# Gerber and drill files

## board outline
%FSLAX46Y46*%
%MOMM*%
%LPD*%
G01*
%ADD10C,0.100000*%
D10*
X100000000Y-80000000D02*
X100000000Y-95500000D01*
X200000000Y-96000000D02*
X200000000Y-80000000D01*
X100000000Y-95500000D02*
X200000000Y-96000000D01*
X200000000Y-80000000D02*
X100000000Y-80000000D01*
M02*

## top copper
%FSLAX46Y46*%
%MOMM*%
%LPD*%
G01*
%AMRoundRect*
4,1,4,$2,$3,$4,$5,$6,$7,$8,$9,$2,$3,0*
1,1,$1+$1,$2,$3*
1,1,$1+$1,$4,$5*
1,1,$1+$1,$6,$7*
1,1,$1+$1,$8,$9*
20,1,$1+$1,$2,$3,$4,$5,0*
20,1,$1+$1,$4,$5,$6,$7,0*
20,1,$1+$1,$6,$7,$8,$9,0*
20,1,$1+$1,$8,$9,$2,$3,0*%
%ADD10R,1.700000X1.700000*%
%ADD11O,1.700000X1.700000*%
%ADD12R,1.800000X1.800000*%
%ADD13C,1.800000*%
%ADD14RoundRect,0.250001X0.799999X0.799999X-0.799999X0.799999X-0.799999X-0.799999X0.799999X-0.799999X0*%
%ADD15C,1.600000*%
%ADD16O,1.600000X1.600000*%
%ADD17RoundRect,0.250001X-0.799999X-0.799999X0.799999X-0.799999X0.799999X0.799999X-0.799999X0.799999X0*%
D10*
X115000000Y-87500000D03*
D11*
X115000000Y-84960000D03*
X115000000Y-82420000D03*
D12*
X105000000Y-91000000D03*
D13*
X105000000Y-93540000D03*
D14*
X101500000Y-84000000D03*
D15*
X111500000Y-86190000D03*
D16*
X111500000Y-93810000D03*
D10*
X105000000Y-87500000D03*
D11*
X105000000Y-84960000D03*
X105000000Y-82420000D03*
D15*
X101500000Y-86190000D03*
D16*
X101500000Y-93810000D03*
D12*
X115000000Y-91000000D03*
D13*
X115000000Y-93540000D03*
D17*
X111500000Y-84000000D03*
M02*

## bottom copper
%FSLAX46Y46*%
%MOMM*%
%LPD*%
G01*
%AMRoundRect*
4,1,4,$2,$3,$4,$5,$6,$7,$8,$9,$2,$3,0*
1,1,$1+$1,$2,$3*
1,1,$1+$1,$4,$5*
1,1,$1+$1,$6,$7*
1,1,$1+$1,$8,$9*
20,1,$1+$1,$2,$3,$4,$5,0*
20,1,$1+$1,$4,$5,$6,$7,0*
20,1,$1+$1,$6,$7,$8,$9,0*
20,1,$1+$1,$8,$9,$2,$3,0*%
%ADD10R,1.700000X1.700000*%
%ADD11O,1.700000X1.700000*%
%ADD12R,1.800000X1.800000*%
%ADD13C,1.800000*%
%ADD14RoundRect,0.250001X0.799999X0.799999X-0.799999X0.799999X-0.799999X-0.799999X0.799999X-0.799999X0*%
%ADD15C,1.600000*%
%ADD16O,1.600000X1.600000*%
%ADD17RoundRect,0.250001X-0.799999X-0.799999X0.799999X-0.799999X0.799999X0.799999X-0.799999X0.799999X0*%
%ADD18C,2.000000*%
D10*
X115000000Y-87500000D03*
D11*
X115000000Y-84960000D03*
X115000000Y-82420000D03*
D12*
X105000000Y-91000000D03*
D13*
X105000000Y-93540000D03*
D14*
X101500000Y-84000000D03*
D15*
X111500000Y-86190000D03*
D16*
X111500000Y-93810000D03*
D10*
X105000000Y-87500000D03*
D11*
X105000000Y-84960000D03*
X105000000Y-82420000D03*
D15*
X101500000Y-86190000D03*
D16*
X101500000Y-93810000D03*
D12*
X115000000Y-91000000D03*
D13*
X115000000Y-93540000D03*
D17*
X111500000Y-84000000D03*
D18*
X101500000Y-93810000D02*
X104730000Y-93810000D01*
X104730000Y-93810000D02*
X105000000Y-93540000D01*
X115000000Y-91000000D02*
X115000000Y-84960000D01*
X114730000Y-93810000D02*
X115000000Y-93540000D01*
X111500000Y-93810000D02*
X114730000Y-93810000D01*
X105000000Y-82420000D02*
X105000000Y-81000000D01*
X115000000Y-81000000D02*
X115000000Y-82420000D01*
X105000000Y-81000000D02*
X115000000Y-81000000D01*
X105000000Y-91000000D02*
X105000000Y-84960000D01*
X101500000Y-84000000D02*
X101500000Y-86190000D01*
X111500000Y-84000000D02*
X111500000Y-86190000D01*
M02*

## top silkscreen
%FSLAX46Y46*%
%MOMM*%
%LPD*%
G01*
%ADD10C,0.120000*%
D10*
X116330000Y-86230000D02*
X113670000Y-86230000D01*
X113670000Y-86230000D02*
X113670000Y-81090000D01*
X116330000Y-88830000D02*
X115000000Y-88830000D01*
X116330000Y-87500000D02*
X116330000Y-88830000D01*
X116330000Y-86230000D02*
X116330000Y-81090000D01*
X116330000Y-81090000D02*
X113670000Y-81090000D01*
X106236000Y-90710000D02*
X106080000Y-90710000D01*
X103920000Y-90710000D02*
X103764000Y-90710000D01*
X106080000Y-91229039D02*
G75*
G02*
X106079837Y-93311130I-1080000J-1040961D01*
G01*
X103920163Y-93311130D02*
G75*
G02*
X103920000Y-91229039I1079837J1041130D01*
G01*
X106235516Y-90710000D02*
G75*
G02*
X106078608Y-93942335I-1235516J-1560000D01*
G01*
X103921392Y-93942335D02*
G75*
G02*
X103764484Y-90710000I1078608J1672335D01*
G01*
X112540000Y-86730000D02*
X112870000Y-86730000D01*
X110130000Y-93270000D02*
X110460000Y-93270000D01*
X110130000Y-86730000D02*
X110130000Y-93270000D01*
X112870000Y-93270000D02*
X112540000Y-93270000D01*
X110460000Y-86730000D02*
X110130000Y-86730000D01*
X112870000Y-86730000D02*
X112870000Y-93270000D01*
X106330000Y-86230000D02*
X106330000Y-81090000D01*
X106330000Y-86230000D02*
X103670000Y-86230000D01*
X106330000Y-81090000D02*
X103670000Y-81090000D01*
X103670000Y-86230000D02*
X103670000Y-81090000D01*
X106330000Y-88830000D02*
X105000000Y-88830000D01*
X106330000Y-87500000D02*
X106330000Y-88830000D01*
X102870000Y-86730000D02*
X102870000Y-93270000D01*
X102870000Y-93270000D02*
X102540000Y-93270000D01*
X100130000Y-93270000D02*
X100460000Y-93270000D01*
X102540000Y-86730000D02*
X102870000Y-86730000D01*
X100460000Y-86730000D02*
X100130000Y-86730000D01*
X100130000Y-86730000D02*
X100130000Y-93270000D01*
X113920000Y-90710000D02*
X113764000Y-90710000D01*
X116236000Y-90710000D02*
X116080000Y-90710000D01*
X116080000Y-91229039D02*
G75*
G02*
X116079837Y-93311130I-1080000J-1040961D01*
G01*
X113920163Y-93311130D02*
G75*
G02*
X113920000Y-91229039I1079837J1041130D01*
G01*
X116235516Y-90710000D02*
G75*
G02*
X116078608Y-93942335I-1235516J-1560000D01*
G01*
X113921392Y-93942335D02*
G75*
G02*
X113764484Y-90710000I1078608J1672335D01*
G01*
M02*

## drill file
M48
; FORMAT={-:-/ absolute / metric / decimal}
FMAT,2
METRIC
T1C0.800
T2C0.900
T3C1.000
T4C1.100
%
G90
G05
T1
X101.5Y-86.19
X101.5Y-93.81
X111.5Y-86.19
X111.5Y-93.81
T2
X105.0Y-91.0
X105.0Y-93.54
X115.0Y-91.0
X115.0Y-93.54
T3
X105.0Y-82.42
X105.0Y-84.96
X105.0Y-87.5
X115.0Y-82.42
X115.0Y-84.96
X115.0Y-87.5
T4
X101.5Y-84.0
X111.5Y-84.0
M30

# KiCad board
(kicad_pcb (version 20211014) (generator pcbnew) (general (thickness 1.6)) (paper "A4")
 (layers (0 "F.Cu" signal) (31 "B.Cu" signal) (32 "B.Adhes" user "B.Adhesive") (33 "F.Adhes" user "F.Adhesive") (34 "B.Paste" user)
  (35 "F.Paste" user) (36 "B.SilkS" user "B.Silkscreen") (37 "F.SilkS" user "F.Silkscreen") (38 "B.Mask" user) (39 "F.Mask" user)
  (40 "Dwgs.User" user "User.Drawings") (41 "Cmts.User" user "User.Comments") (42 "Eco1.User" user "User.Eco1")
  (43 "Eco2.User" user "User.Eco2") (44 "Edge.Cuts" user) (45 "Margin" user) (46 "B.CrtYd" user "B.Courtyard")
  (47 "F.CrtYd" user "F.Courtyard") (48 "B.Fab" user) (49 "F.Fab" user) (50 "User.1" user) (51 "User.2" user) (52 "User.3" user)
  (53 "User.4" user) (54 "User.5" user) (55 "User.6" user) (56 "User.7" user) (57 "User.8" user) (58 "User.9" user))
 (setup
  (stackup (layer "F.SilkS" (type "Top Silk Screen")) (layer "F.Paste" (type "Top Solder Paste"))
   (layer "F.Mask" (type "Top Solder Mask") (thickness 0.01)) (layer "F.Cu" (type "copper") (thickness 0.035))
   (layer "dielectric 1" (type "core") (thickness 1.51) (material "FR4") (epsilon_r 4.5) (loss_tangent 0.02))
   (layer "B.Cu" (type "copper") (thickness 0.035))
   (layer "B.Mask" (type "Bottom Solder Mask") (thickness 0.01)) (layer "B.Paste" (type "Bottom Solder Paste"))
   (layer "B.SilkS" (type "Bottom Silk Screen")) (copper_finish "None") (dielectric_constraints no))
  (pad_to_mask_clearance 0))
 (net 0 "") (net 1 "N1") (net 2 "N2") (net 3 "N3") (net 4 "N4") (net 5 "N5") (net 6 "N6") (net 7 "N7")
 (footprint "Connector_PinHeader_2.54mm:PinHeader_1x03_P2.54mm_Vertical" (layer "F.Cu") (at 115 87.5 180)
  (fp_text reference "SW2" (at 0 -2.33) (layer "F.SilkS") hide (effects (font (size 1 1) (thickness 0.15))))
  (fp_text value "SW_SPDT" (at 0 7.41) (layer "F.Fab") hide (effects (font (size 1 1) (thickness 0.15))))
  (fp_line (start -1.33 1.27) (end 1.33 1.27) (layer "F.SilkS") (width 0.12))
  (fp_line (start 1.33 1.27) (end 1.33 6.41) (layer "F.SilkS") (width 0.12))
  (fp_line (start -1.33 -1.33) (end 0 -1.33) (layer "F.SilkS") (width 0.12))
  (fp_line (start -1.33 0) (end -1.33 -1.33) (layer "F.SilkS") (width 0.12))
  (fp_line (start -1.33 1.27) (end -1.33 6.41) (layer "F.SilkS") (width 0.12))
  (fp_line (start -1.33 6.41) (end 1.33 6.41) (layer "F.SilkS") (width 0.12))
  (pad "1" thru_hole rect (at 0 0 180) (size 1.7 1.7) (drill 1) (layers *.Cu *.Mask) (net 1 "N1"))
  (pad "2" thru_hole oval (at 0 2.54 180) (size 1.7 1.7) (drill 1) (layers *.Cu *.Mask) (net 1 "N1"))
  (pad "3" thru_hole oval (at 0 5.08 180) (size 1.7 1.7) (drill 1) (layers *.Cu *.Mask) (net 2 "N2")))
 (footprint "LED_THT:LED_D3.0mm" (layer "F.Cu") (at 105 91 -90)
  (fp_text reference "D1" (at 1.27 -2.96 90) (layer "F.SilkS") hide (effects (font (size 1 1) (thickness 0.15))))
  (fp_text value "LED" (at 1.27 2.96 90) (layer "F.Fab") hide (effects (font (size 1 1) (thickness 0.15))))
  (fp_line (start -0.29 -1.236) (end -0.29 -1.08) (layer "F.SilkS") (width 0.12))
  (fp_line (start -0.29 1.08) (end -0.29 1.236) (layer "F.SilkS") (width 0.12))
  (fp_arc (start 0.229039 -1.08) (mid 1.270117 -1.5) (end 2.31113 -1.079837) (layer "F.SilkS") (width 0.12))
  (fp_arc (start 2.31113 1.079837) (mid 1.270117 1.5) (end 0.229039 1.08) (layer "F.SilkS") (width 0.12))
  (fp_arc (start -0.29 -1.235516) (mid 1.366487 -1.987659) (end 2.942335 -1.078608) (layer "F.SilkS") (width 0.12))
  (fp_arc (start 2.942335 1.078608) (mid 1.366487 1.987659) (end -0.29 1.235516) (layer "F.SilkS") (width 0.12))
  (pad "1" thru_hole rect (at 0 0 270) (size 1.8 1.8) (drill 0.9) (layers *.Cu *.Mask) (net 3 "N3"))
  (pad "2" thru_hole circle (at 2.54 0 270) (size 1.8 1.8) (drill 0.9) (layers *.Cu *.Mask) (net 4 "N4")))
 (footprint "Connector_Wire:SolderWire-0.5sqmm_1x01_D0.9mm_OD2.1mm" (layer "F.Cu") (at 101.5 84 180)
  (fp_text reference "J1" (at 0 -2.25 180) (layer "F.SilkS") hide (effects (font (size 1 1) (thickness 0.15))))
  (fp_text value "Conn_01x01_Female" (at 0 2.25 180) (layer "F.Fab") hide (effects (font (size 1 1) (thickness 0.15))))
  (pad "1" thru_hole roundrect (at 0 0 180) (size 2.1 2.1) (drill 1.1) (layers *.Cu *.Mask) (roundrect_rratio 0.119048) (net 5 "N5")))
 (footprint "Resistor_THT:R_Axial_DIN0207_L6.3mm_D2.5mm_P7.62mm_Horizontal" (layer "F.Cu") (at 111.5 86.19 -90)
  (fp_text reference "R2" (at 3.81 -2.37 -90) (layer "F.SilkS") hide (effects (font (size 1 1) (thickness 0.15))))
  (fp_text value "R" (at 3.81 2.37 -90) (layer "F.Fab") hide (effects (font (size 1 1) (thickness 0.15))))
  (fp_line (start 0.54 -1.04) (end 0.54 -1.37) (layer "F.SilkS") (width 0.12))
  (fp_line (start 7.08 1.37) (end 7.08 1.04) (layer "F.SilkS") (width 0.12))
  (fp_line (start 0.54 1.37) (end 7.08 1.37) (layer "F.SilkS") (width 0.12))
  (fp_line (start 7.08 -1.37) (end 7.08 -1.04) (layer "F.SilkS") (width 0.12))
  (fp_line (start 0.54 1.04) (end 0.54 1.37) (layer "F.SilkS") (width 0.12))
  (fp_line (start 0.54 -1.37) (end 7.08 -1.37) (layer "F.SilkS") (width 0.12))
  (pad "1" thru_hole circle (at 0 0 270) (size 1.6 1.6) (drill 0.8) (layers *.Cu *.Mask) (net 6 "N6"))
  (pad "2" thru_hole oval (at 7.62 0 270) (size 1.6 1.6) (drill 0.8) (layers *.Cu *.Mask) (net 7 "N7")))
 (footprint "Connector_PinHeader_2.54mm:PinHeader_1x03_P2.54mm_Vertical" (layer "F.Cu") (at 105 87.5 180)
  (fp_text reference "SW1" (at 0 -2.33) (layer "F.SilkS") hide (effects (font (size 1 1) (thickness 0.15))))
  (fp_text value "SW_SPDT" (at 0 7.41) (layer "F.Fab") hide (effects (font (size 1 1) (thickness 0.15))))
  (fp_line (start -1.33 1.27) (end -1.33 6.41) (layer "F.SilkS") (width 0.12))
  (fp_line (start -1.33 1.27) (end 1.33 1.27) (layer "F.SilkS") (width 0.12))
  (fp_line (start -1.33 6.41) (end 1.33 6.41) (layer "F.SilkS") (width 0.12))
  (fp_line (start 1.33 1.27) (end 1.33 6.41) (layer "F.SilkS") (width 0.12))
  (fp_line (start -1.33 -1.33) (end 0 -1.33) (layer "F.SilkS") (width 0.12))
  (fp_line (start -1.33 0) (end -1.33 -1.33) (layer "F.SilkS") (width 0.12))
  (pad "1" thru_hole rect (at 0 0 180) (size 1.7 1.7) (drill 1) (layers *.Cu *.Mask) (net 3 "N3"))
  (pad "2" thru_hole oval (at 0 2.54 180) (size 1.7 1.7) (drill 1) (layers *.Cu *.Mask) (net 3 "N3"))
  (pad "3" thru_hole oval (at 0 5.08 180) (size 1.7 1.7) (drill 1) (layers *.Cu *.Mask) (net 2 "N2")))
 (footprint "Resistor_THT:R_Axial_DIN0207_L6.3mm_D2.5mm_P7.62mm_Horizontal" (layer "F.Cu") (at 101.5 86.19 -90)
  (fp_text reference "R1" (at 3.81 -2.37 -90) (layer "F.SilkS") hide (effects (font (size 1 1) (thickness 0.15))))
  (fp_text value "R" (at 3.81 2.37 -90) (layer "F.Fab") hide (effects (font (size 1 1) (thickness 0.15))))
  (fp_line (start 0.54 -1.37) (end 7.08 -1.37) (layer "F.SilkS") (width 0.12))
  (fp_line (start 7.08 -1.37) (end 7.08 -1.04) (layer "F.SilkS") (width 0.12))
  (fp_line (start 7.08 1.37) (end 7.08 1.04) (layer "F.SilkS") (width 0.12))
  (fp_line (start 0.54 -1.04) (end 0.54 -1.37) (layer "F.SilkS") (width 0.12))
  (fp_line (start 0.54 1.04) (end 0.54 1.37) (layer "F.SilkS") (width 0.12))
  (fp_line (start 0.54 1.37) (end 7.08 1.37) (layer "F.SilkS") (width 0.12))
  (pad "1" thru_hole circle (at 0 0 270) (size 1.6 1.6) (drill 0.8) (layers *.Cu *.Mask) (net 5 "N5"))
  (pad "2" thru_hole oval (at 7.62 0 270) (size 1.6 1.6) (drill 0.8) (layers *.Cu *.Mask) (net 4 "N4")))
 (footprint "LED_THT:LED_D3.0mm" (layer "F.Cu") (at 115 91 -90)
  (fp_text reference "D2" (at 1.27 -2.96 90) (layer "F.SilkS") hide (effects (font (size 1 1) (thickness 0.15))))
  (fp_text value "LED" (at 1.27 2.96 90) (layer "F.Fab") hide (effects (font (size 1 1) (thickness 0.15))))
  (fp_line (start -0.29 1.08) (end -0.29 1.236) (layer "F.SilkS") (width 0.12))
  (fp_line (start -0.29 -1.236) (end -0.29 -1.08) (layer "F.SilkS") (width 0.12))
  (fp_arc (start 0.229039 -1.08) (mid 1.270117 -1.5) (end 2.31113 -1.079837) (layer "F.SilkS") (width 0.12))
  (fp_arc (start 2.31113 1.079837) (mid 1.270117 1.5) (end 0.229039 1.08) (layer "F.SilkS") (width 0.12))
  (fp_arc (start -0.29 -1.235516) (mid 1.366487 -1.987659) (end 2.942335 -1.078608) (layer "F.SilkS") (width 0.12))
  (fp_arc (start 2.942335 1.078608) (mid 1.366487 1.987659) (end -0.29 1.235516) (layer "F.SilkS") (width 0.12))
  (pad "1" thru_hole rect (at 0 0 270) (size 1.8 1.8) (drill 0.9) (layers *.Cu *.Mask) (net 1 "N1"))
  (pad "2" thru_hole circle (at 2.54 0 270) (size 1.8 1.8) (drill 0.9) (layers *.Cu *.Mask) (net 7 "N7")))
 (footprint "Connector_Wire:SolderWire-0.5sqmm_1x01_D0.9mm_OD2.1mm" (layer "F.Cu") (at 111.5 84)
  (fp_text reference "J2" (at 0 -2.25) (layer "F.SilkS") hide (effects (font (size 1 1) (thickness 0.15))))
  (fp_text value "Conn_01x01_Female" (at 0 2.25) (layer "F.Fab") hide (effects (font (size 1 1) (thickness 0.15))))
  (pad "1" thru_hole roundrect (at 0 0) (size 2.1 2.1) (drill 1.1) (layers *.Cu *.Mask) (roundrect_rratio 0.119048) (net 6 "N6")))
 (gr_line (start 100 80) (end 100 95.5) (layer "Edge.Cuts") (width 0.1))
 (gr_line (start 200 96) (end 200 80) (layer "Edge.Cuts") (width 0.1))
 (gr_line (start 100 95.5) (end 200 96) (layer "Edge.Cuts") (width 0.1))
 (gr_line (start 200 80) (end 100 80) (layer "Edge.Cuts") (width 0.1))
 (segment (start 101.5 93.81) (end 104.73 93.81) (width 2) (layer "B.Cu") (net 4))
 (segment (start 104.73 93.81) (end 105 93.54) (width 2) (layer "B.Cu") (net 4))
 (segment (start 115 91) (end 115 84.96) (width 2) (layer "B.Cu") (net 1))
 (segment (start 114.73 93.81) (end 115 93.54) (width 2) (layer "B.Cu") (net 7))
 (segment (start 111.5 93.81) (end 114.73 93.81) (width 2) (layer "B.Cu") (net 7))
 (segment (start 105 82.42) (end 105 81) (width 2) (layer "B.Cu") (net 2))
 (segment (start 115 81) (end 115 82.42) (width 2) (layer "B.Cu") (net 2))
 (segment (start 105 81) (end 115 81) (width 2) (layer "B.Cu") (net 2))
 (segment (start 105 91) (end 105 84.96) (width 2) (layer "B.Cu") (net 3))
 (segment (start 101.5 84) (end 101.5 86.19) (width 2) (layer "B.Cu") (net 5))
 (segment (start 111.5 84) (end 111.5 86.19) (width 2) (layer "B.Cu") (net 6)))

